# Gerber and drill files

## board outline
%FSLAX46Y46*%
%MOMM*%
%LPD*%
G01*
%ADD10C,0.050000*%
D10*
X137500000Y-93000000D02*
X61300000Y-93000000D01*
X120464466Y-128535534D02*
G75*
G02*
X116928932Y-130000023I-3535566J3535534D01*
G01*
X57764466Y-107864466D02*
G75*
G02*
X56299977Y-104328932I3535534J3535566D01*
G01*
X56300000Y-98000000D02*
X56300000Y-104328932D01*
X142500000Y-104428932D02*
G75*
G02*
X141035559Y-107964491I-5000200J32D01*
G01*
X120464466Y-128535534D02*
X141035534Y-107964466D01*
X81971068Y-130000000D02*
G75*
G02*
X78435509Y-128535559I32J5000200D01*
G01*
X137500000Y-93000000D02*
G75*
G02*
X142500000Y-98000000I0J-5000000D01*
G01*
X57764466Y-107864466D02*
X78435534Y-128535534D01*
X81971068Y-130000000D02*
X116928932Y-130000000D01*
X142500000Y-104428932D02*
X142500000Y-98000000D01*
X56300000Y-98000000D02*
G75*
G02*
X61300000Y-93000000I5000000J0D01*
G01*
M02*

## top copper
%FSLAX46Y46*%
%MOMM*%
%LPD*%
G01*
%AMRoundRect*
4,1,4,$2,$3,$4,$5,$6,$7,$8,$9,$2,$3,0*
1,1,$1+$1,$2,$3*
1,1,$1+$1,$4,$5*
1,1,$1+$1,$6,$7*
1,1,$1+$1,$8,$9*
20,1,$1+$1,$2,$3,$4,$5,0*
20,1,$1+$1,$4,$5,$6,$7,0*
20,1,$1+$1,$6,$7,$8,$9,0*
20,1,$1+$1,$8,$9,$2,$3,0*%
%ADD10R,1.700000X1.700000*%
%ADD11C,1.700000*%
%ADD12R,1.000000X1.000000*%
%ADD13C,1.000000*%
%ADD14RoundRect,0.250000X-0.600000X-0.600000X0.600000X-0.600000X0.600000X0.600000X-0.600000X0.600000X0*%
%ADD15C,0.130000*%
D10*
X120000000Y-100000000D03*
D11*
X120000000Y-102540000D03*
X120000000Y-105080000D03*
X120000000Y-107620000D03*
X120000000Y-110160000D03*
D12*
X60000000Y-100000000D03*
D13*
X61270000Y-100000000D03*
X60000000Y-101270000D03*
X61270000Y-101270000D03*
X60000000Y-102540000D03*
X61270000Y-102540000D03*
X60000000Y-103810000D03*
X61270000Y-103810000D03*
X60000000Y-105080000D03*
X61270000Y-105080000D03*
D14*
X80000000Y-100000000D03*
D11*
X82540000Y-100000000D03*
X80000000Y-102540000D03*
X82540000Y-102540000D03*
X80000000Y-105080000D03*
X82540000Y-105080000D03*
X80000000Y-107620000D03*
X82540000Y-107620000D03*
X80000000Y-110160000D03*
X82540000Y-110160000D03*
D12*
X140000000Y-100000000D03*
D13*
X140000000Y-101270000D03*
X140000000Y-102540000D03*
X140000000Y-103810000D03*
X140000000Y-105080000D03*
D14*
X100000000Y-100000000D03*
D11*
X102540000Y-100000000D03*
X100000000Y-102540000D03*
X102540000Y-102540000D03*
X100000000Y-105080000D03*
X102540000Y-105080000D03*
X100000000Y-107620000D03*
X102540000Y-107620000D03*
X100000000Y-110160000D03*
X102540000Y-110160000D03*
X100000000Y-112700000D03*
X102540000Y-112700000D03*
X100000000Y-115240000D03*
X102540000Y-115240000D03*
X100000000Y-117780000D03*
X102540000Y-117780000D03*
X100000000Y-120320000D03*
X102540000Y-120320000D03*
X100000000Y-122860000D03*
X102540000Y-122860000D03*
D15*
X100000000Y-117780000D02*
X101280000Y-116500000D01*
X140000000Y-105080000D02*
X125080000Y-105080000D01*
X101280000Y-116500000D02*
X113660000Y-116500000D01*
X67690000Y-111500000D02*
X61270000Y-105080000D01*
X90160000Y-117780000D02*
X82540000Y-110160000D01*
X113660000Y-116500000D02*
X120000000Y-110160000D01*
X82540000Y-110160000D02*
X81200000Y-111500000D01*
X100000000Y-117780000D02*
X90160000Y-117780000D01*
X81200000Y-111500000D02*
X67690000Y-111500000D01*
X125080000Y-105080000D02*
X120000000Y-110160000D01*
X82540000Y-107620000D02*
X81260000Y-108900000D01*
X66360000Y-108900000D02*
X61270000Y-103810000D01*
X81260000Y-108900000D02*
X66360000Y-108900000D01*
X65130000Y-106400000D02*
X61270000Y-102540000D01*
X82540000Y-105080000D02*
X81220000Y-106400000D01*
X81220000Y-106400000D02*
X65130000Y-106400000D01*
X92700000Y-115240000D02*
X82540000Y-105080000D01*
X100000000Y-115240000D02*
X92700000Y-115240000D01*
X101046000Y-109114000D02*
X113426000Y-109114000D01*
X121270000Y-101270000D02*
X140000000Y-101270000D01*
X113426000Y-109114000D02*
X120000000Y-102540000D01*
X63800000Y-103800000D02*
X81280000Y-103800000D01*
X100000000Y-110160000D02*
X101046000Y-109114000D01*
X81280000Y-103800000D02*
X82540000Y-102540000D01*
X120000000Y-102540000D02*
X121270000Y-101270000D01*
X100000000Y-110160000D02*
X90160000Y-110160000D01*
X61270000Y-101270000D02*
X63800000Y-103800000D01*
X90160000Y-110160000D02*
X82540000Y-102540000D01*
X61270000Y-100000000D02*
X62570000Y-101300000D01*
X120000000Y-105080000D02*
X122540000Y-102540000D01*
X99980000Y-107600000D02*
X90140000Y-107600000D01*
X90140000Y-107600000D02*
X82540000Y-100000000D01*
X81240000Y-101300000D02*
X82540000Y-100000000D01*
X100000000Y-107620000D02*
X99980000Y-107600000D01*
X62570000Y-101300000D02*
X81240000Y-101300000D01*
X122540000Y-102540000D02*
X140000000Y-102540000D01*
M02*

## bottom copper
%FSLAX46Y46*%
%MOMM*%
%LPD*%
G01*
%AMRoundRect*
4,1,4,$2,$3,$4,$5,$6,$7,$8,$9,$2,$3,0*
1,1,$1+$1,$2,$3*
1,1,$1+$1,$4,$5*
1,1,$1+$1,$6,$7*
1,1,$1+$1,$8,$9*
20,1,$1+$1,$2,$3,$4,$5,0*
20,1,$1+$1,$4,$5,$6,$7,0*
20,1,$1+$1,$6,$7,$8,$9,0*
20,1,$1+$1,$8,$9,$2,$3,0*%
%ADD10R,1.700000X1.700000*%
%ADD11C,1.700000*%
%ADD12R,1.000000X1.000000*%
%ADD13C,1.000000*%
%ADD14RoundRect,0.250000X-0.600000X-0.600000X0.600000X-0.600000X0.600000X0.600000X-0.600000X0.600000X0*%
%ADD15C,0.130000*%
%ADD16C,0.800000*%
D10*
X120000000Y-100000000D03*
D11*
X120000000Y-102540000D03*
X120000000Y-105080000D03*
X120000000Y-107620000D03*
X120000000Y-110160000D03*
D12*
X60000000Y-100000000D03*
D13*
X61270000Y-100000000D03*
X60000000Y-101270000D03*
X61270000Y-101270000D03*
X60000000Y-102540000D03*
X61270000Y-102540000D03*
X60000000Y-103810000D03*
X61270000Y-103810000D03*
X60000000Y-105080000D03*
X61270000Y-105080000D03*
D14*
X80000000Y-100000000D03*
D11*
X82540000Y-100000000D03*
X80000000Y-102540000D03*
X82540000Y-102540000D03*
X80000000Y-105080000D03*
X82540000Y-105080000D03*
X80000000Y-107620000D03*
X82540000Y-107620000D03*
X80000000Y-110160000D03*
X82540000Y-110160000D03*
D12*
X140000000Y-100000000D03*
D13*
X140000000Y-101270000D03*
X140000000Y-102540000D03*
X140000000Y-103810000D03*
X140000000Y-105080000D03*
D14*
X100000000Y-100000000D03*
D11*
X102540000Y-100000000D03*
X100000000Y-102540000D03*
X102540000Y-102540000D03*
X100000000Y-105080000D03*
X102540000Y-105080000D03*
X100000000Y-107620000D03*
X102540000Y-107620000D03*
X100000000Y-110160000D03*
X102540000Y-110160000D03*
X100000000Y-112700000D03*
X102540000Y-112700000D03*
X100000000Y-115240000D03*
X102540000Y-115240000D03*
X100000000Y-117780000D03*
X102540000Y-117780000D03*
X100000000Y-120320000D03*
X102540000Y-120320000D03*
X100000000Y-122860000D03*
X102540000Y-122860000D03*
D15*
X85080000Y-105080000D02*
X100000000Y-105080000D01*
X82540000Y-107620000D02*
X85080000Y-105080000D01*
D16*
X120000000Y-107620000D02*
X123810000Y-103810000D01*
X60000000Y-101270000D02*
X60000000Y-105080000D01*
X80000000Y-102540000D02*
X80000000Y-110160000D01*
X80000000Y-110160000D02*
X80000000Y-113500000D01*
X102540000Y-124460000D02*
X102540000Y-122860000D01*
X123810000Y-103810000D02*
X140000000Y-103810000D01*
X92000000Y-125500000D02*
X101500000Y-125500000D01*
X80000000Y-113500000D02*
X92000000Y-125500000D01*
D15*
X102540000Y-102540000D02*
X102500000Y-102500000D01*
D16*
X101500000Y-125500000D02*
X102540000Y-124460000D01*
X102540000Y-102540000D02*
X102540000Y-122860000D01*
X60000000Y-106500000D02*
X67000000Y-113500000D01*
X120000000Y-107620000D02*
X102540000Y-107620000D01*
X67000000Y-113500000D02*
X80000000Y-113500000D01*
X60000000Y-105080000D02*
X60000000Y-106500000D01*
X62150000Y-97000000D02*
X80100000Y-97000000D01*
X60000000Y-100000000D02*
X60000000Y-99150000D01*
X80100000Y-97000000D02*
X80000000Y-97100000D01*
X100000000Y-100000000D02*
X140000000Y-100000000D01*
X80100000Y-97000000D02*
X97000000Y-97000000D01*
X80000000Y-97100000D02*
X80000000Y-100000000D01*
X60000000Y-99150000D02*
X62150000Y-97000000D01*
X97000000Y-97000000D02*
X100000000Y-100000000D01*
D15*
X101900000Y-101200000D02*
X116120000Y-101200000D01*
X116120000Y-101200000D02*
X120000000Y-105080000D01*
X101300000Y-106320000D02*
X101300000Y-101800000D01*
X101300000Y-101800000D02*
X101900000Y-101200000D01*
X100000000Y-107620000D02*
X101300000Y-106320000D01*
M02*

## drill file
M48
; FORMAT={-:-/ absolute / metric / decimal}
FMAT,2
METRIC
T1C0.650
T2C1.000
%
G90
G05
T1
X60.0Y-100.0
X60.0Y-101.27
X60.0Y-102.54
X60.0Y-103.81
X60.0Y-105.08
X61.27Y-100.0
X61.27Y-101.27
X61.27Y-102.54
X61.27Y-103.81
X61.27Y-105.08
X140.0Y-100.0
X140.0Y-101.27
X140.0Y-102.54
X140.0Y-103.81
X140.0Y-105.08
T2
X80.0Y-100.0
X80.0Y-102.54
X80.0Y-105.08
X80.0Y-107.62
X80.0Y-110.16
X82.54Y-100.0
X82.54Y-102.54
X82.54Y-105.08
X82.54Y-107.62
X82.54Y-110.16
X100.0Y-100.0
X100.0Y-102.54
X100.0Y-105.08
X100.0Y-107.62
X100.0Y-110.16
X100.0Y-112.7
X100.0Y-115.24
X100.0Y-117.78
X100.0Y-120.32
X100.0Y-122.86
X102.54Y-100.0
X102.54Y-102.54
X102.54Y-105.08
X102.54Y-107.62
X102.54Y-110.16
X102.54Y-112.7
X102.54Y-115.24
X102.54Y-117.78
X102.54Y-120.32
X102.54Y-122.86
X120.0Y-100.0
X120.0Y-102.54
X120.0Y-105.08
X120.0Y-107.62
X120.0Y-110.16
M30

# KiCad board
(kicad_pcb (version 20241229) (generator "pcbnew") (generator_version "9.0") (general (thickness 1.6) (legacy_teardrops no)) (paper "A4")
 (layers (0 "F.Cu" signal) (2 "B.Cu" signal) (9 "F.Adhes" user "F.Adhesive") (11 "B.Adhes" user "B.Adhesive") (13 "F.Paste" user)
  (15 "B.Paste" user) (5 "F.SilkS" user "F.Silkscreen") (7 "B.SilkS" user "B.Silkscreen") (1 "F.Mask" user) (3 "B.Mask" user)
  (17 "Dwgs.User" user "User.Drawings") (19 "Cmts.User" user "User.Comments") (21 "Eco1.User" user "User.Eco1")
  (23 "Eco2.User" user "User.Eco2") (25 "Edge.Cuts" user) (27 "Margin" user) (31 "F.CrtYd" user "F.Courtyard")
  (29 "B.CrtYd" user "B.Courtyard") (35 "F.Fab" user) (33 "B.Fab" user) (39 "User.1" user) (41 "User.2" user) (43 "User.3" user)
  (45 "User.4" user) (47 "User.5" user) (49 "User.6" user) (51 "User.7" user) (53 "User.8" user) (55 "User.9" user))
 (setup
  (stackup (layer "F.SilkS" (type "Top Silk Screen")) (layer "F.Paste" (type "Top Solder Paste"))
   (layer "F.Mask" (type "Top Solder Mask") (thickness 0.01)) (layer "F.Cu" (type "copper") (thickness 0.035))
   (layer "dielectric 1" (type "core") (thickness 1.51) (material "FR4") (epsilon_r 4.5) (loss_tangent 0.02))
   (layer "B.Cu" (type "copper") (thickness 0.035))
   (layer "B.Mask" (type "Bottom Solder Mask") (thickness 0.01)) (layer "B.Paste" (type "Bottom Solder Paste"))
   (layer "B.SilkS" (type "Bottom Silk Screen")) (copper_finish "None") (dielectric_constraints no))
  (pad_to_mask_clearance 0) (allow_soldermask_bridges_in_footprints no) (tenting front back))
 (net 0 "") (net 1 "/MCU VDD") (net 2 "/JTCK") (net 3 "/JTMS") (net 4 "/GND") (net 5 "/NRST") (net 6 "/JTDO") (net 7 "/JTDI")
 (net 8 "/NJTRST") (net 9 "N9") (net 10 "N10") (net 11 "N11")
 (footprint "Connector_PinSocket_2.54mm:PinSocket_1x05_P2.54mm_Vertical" (layer "F.Cu") (at 120 100)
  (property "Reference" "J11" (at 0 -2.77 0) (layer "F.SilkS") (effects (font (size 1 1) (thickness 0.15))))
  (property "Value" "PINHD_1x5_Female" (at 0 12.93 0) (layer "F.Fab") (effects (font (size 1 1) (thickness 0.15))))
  (pad "1" thru_hole rect (at 0 0) (size 1.7 1.7) (drill 1) (layers "*.Cu" "*.Mask") (remove_unused_layers no) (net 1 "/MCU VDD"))
  (pad "2" thru_hole circle (at 0 2.54) (size 1.7 1.7) (drill 1) (layers "*.Cu" "*.Mask") (remove_unused_layers no) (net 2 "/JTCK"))
  (pad "3" thru_hole circle (at 0 5.08) (size 1.7 1.7) (drill 1) (layers "*.Cu" "*.Mask") (remove_unused_layers no) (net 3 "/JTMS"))
  (pad "4" thru_hole circle (at 0 7.62) (size 1.7 1.7) (drill 1) (layers "*.Cu" "*.Mask") (remove_unused_layers no) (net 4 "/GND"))
  (pad "5" thru_hole circle (at 0 10.16) (size 1.7 1.7) (drill 1) (layers "*.Cu" "*.Mask") (remove_unused_layers no) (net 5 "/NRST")))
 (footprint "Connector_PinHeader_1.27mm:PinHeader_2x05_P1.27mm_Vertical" (layer "F.Cu") (at 60 100)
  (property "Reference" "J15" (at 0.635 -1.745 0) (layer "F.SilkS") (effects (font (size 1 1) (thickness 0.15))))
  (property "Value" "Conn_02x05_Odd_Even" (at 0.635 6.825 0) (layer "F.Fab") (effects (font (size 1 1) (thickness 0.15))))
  (pad "1" thru_hole rect (at 0 0) (size 1 1) (drill 0.65) (layers "*.Cu" "*.Mask") (remove_unused_layers no) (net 1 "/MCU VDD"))
  (pad "2" thru_hole circle (at 1.27 0) (size 1 1) (drill 0.65) (layers "*.Cu" "*.Mask") (remove_unused_layers no) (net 3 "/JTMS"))
  (pad "3" thru_hole circle (at 0 1.27) (size 1 1) (drill 0.65) (layers "*.Cu" "*.Mask") (remove_unused_layers no) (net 4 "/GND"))
  (pad "4" thru_hole circle (at 1.27 1.27) (size 1 1) (drill 0.65) (layers "*.Cu" "*.Mask") (remove_unused_layers no) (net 2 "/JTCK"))
  (pad "5" thru_hole circle (at 0 2.54) (size 1 1) (drill 0.65) (layers "*.Cu" "*.Mask") (remove_unused_layers no) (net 4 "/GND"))
  (pad "6" thru_hole circle (at 1.27 2.54) (size 1 1) (drill 0.65) (layers "*.Cu" "*.Mask") (remove_unused_layers no) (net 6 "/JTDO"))
  (pad "7" thru_hole circle (at 0 3.81) (size 1 1) (drill 0.65) (layers "*.Cu" "*.Mask") (remove_unused_layers no) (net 4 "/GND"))
  (pad "8" thru_hole circle (at 1.27 3.81) (size 1 1) (drill 0.65) (layers "*.Cu" "*.Mask") (remove_unused_layers no) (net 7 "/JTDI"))
  (pad "9" thru_hole circle (at 0 5.08) (size 1 1) (drill 0.65) (layers "*.Cu" "*.Mask") (remove_unused_layers no) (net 4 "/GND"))
  (pad "10" thru_hole circle (at 1.27 5.08) (size 1 1) (drill 0.65) (layers "*.Cu" "*.Mask") (remove_unused_layers no) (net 5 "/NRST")))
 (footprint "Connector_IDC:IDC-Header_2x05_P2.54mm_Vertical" (layer "F.Cu") (at 80 100)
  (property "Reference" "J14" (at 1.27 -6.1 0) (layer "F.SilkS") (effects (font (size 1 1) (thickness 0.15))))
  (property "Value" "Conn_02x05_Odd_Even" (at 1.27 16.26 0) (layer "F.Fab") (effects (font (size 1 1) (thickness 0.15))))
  (pad "1" thru_hole roundrect (at 0 0) (size 1.7 1.7) (drill 1) (layers "*.Cu" "*.Mask") (remove_unused_layers no)
   (roundrect_rratio 0.147059) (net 1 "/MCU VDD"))
  (pad "2" thru_hole circle (at 2.54 0) (size 1.7 1.7) (drill 1) (layers "*.Cu" "*.Mask") (remove_unused_layers no) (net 3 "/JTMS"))
  (pad "3" thru_hole circle (at 0 2.54) (size 1.7 1.7) (drill 1) (layers "*.Cu" "*.Mask") (remove_unused_layers no) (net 4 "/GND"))
  (pad "4" thru_hole circle (at 2.54 2.54) (size 1.7 1.7) (drill 1) (layers "*.Cu" "*.Mask") (remove_unused_layers no) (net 2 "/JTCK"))
  (pad "5" thru_hole circle (at 0 5.08) (size 1.7 1.7) (drill 1) (layers "*.Cu" "*.Mask") (remove_unused_layers no) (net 4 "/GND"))
  (pad "6" thru_hole circle (at 2.54 5.08) (size 1.7 1.7) (drill 1) (layers "*.Cu" "*.Mask") (remove_unused_layers no) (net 6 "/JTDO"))
  (pad "7" thru_hole circle (at 0 7.62) (size 1.7 1.7) (drill 1) (layers "*.Cu" "*.Mask") (remove_unused_layers no) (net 4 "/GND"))
  (pad "8" thru_hole circle (at 2.54 7.62) (size 1.7 1.7) (drill 1) (layers "*.Cu" "*.Mask") (remove_unused_layers no) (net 7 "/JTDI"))
  (pad "9" thru_hole circle (at 0 10.16) (size 1.7 1.7) (drill 1) (layers "*.Cu" "*.Mask") (remove_unused_layers no) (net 4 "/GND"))
  (pad "10" thru_hole circle (at 2.54 10.16) (size 1.7 1.7) (drill 1) (layers "*.Cu" "*.Mask") (remove_unused_layers no) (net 5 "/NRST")))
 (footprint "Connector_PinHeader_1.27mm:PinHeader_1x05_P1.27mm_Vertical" (layer "F.Cu") (at 140 100)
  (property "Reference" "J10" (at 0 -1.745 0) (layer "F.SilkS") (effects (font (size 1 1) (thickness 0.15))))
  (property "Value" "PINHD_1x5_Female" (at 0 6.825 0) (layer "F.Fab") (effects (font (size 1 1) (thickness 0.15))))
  (pad "1" thru_hole rect (at 0 0) (size 1 1) (drill 0.65) (layers "*.Cu" "*.Mask") (remove_unused_layers no) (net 1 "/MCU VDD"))
  (pad "2" thru_hole circle (at 0 1.27) (size 1 1) (drill 0.65) (layers "*.Cu" "*.Mask") (remove_unused_layers no) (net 2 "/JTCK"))
  (pad "3" thru_hole circle (at 0 2.54) (size 1 1) (drill 0.65) (layers "*.Cu" "*.Mask") (remove_unused_layers no) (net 3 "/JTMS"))
  (pad "4" thru_hole circle (at 0 3.81) (size 1 1) (drill 0.65) (layers "*.Cu" "*.Mask") (remove_unused_layers no) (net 4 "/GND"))
  (pad "5" thru_hole circle (at 0 5.08) (size 1 1) (drill 0.65) (layers "*.Cu" "*.Mask") (remove_unused_layers no) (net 5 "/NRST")))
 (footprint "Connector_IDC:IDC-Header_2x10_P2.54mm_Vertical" (layer "F.Cu") (at 100 100)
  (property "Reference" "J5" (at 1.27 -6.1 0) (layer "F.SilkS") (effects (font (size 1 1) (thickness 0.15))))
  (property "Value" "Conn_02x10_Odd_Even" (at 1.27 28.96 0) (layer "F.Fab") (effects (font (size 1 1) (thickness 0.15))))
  (pad "1" thru_hole roundrect (at 0 0) (size 1.7 1.7) (drill 1) (layers "*.Cu" "*.Mask") (remove_unused_layers no)
   (roundrect_rratio 0.147059) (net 1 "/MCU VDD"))
  (pad "2" thru_hole circle (at 2.54 0) (size 1.7 1.7) (drill 1) (layers "*.Cu" "*.Mask") (remove_unused_layers no) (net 1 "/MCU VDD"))
  (pad "3" thru_hole circle (at 0 2.54) (size 1.7 1.7) (drill 1) (layers "*.Cu" "*.Mask") (remove_unused_layers no) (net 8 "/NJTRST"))
  (pad "4" thru_hole circle (at 2.54 2.54) (size 1.7 1.7) (drill 1) (layers "*.Cu" "*.Mask") (remove_unused_layers no) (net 4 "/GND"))
  (pad "5" thru_hole circle (at 0 5.08) (size 1.7 1.7) (drill 1) (layers "*.Cu" "*.Mask") (remove_unused_layers no) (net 7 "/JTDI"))
  (pad "6" thru_hole circle (at 2.54 5.08) (size 1.7 1.7) (drill 1) (layers "*.Cu" "*.Mask") (remove_unused_layers no) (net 4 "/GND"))
  (pad "7" thru_hole circle (at 0 7.62) (size 1.7 1.7) (drill 1) (layers "*.Cu" "*.Mask") (remove_unused_layers no) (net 3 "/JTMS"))
  (pad "8" thru_hole circle (at 2.54 7.62) (size 1.7 1.7) (drill 1) (layers "*.Cu" "*.Mask") (remove_unused_layers no) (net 4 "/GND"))
  (pad "9" thru_hole circle (at 0 10.16) (size 1.7 1.7) (drill 1) (layers "*.Cu" "*.Mask") (remove_unused_layers no) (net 2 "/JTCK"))
  (pad "10" thru_hole circle (at 2.54 10.16) (size 1.7 1.7) (drill 1) (layers "*.Cu" "*.Mask") (remove_unused_layers no) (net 4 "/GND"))
  (pad "11" thru_hole circle (at 0 12.7) (size 1.7 1.7) (drill 1) (layers "*.Cu" "*.Mask") (remove_unused_layers no) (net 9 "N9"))
  (pad "12" thru_hole circle (at 2.54 12.7) (size 1.7 1.7) (drill 1) (layers "*.Cu" "*.Mask") (remove_unused_layers no) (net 4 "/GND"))
  (pad "13" thru_hole circle (at 0 15.24) (size 1.7 1.7) (drill 1) (layers "*.Cu" "*.Mask") (remove_unused_layers no) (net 6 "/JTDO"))
  (pad "14" thru_hole circle (at 2.54 15.24) (size 1.7 1.7) (drill 1) (layers "*.Cu" "*.Mask") (remove_unused_layers no) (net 4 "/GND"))
  (pad "15" thru_hole circle (at 0 17.78) (size 1.7 1.7) (drill 1) (layers "*.Cu" "*.Mask") (remove_unused_layers no) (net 5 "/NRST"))
  (pad "16" thru_hole circle (at 2.54 17.78) (size 1.7 1.7) (drill 1) (layers "*.Cu" "*.Mask") (remove_unused_layers no) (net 4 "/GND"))
  (pad "17" thru_hole circle (at 0 20.32) (size 1.7 1.7) (drill 1) (layers "*.Cu" "*.Mask") (remove_unused_layers no) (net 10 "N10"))
  (pad "18" thru_hole circle (at 2.54 20.32) (size 1.7 1.7) (drill 1) (layers "*.Cu" "*.Mask") (remove_unused_layers no) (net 4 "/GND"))
  (pad "19" thru_hole circle (at 0 22.86) (size 1.7 1.7) (drill 1) (layers "*.Cu" "*.Mask") (remove_unused_layers no) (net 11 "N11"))
  (pad "20" thru_hole circle (at 2.54 22.86) (size 1.7 1.7) (drill 1) (layers "*.Cu" "*.Mask") (remove_unused_layers no) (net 4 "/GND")))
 (gr_line (start 137.5 93) (end 61.3 93) (stroke (width 0.05) (type default)) (layer "Edge.Cuts"))
 (gr_arc (start 120.464466 128.535534) (mid 118.842349 129.619398) (end 116.928932 130) (stroke (width 0.05) (type default))
  (layer "Edge.Cuts"))
 (gr_arc (start 57.764466 107.864466) (mid 56.680602 106.242349) (end 56.3 104.328932) (stroke (width 0.05) (type default))
  (layer "Edge.Cuts"))
 (gr_line (start 56.3 98) (end 56.3 104.328932) (stroke (width 0.05) (type default)) (layer "Edge.Cuts"))
 (gr_arc (start 142.5 104.428932) (mid 142.119387 106.342342) (end 141.035534 107.964466) (stroke (width 0.05) (type default))
  (layer "Edge.Cuts"))
 (gr_line (start 120.464466 128.535534) (end 141.035534 107.964466) (stroke (width 0.05) (type default)) (layer "Edge.Cuts"))
 (gr_arc (start 81.971068 130) (mid 80.057658 129.619387) (end 78.435534 128.535534) (stroke (width 0.05) (type default))
  (layer "Edge.Cuts"))
 (gr_arc (start 137.5 93) (mid 141.035534 94.464466) (end 142.5 98) (stroke (width 0.05) (type default)) (layer "Edge.Cuts"))
 (gr_line (start 57.764466 107.864466) (end 78.435534 128.535534) (stroke (width 0.05) (type default)) (layer "Edge.Cuts"))
 (gr_line (start 81.971068 130) (end 116.928932 130) (stroke (width 0.05) (type default)) (layer "Edge.Cuts"))
 (gr_line (start 142.5 104.428932) (end 142.5 98) (stroke (width 0.05) (type default)) (layer "Edge.Cuts"))
 (gr_arc (start 56.3 98) (mid 57.764466 94.464466) (end 61.3 93) (stroke (width 0.05) (type default)) (layer "Edge.Cuts"))
 (segment (start 100 117.78) (end 101.28 116.5) (width 0.13) (layer "F.Cu") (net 5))
 (segment (start 140 105.08) (end 125.08 105.08) (width 0.13) (layer "F.Cu") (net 5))
 (segment (start 101.28 116.5) (end 113.66 116.5) (width 0.13) (layer "F.Cu") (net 5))
 (segment (start 67.69 111.5) (end 61.27 105.08) (width 0.13) (layer "F.Cu") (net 5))
 (segment (start 90.16 117.78) (end 82.54 110.16) (width 0.13) (layer "F.Cu") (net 5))
 (segment (start 113.66 116.5) (end 120 110.16) (width 0.13) (layer "F.Cu") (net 5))
 (segment (start 82.54 110.16) (end 81.2 111.5) (width 0.13) (layer "F.Cu") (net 5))
 (segment (start 100 117.78) (end 90.16 117.78) (width 0.13) (layer "F.Cu") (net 5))
 (segment (start 81.2 111.5) (end 67.69 111.5) (width 0.13) (layer "F.Cu") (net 5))
 (segment (start 125.08 105.08) (end 120 110.16) (width 0.13) (layer "F.Cu") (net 5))
 (segment (start 82.54 107.62) (end 81.26 108.9) (width 0.13) (layer "F.Cu") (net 7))
 (segment (start 66.36 108.9) (end 61.27 103.81) (width 0.13) (layer "F.Cu") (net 7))
 (segment (start 81.26 108.9) (end 66.36 108.9) (width 0.13) (layer "F.Cu") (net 7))
 (segment (start 85.08 105.08) (end 100 105.08) (width 0.13) (layer "B.Cu") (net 7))
 (segment (start 82.54 107.62) (end 85.08 105.08) (width 0.13) (layer "B.Cu") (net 7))
 (segment (start 120 107.62) (end 123.81 103.81) (width 0.8) (layer "B.Cu") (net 4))
 (segment (start 60 101.27) (end 60 105.08) (width 0.8) (layer "B.Cu") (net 4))
 (segment (start 80 102.54) (end 80 110.16) (width 0.8) (layer "B.Cu") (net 4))
 (segment (start 80 110.16) (end 80 113.5) (width 0.8) (layer "B.Cu") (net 4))
 (segment (start 102.54 124.46) (end 102.54 122.86) (width 0.8) (layer "B.Cu") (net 4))
 (segment (start 123.81 103.81) (end 140 103.81) (width 0.8) (layer "B.Cu") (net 4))
 (segment (start 92 125.5) (end 101.5 125.5) (width 0.8) (layer "B.Cu") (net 4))
 (segment (start 80 113.5) (end 92 125.5) (width 0.8) (layer "B.Cu") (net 4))
 (segment (start 102.54 102.54) (end 102.5 102.5) (width 0.13) (layer "B.Cu") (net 4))
 (segment (start 101.5 125.5) (end 102.54 124.46) (width 0.8) (layer "B.Cu") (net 4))
 (segment (start 102.54 102.54) (end 102.54 122.86) (width 0.8) (layer "B.Cu") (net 4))
 (segment (start 60 106.5) (end 67 113.5) (width 0.8) (layer "B.Cu") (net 4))
 (segment (start 120 107.62) (end 102.54 107.62) (width 0.8) (layer "B.Cu") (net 4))
 (segment (start 67 113.5) (end 80 113.5) (width 0.8) (layer "B.Cu") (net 4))
 (segment (start 60 105.08) (end 60 106.5) (width 0.8) (layer "B.Cu") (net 4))
 (segment (start 65.13 106.4) (end 61.27 102.54) (width 0.13) (layer "F.Cu") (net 6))
 (segment (start 82.54 105.08) (end 81.22 106.4) (width 0.13) (layer "F.Cu") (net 6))
 (segment (start 81.22 106.4) (end 65.13 106.4) (width 0.13) (layer "F.Cu") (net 6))
 (segment (start 92.7 115.24) (end 82.54 105.08) (width 0.13) (layer "F.Cu") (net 6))
 (segment (start 100 115.24) (end 92.7 115.24) (width 0.13) (layer "F.Cu") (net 6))
 (segment (start 101.046 109.114) (end 113.426 109.114) (width 0.13) (layer "F.Cu") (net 2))
 (segment (start 121.27 101.27) (end 140 101.27) (width 0.13) (layer "F.Cu") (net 2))
 (segment (start 113.426 109.114) (end 120 102.54) (width 0.13) (layer "F.Cu") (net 2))
 (segment (start 63.8 103.8) (end 81.28 103.8) (width 0.13) (layer "F.Cu") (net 2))
 (segment (start 100 110.16) (end 101.046 109.114) (width 0.13) (layer "F.Cu") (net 2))
 (segment (start 81.28 103.8) (end 82.54 102.54) (width 0.13) (layer "F.Cu") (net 2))
 (segment (start 120 102.54) (end 121.27 101.27) (width 0.13) (layer "F.Cu") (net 2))
 (segment (start 100 110.16) (end 90.16 110.16) (width 0.13) (layer "F.Cu") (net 2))
 (segment (start 61.27 101.27) (end 63.8 103.8) (width 0.13) (layer "F.Cu") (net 2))
 (segment (start 90.16 110.16) (end 82.54 102.54) (width 0.13) (layer "F.Cu") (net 2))
 (segment (start 62.15 97) (end 80.1 97) (width 0.8) (layer "B.Cu") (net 1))
 (segment (start 60 100) (end 60 99.15) (width 0.8) (layer "B.Cu") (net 1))
 (segment (start 80.1 97) (end 80 97.1) (width 0.8) (layer "B.Cu") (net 1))
 (segment (start 100 100) (end 140 100) (width 0.8) (layer "B.Cu") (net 1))
 (segment (start 80.1 97) (end 97 97) (width 0.8) (layer "B.Cu") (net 1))
 (segment (start 80 97.1) (end 80 100) (width 0.8) (layer "B.Cu") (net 1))
 (segment (start 60 99.15) (end 62.15 97) (width 0.8) (layer "B.Cu") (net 1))
 (segment (start 97 97) (end 100 100) (width 0.8) (layer "B.Cu") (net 1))
 (segment (start 61.27 100) (end 62.57 101.3) (width 0.13) (layer "F.Cu") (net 3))
 (segment (start 120 105.08) (end 122.54 102.54) (width 0.13) (layer "F.Cu") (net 3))
 (segment (start 99.98 107.6) (end 90.14 107.6) (width 0.13) (layer "F.Cu") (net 3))
 (segment (start 90.14 107.6) (end 82.54 100) (width 0.13) (layer "F.Cu") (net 3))
 (segment (start 81.24 101.3) (end 82.54 100) (width 0.13) (layer "F.Cu") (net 3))
 (segment (start 100 107.62) (end 99.98 107.6) (width 0.13) (layer "F.Cu") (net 3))
 (segment (start 62.57 101.3) (end 81.24 101.3) (width 0.13) (layer "F.Cu") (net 3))
 (segment (start 122.54 102.54) (end 140 102.54) (width 0.13) (layer "F.Cu") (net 3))
 (segment (start 101.9 101.2) (end 116.12 101.2) (width 0.13) (layer "B.Cu") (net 3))
 (segment (start 116.12 101.2) (end 120 105.08) (width 0.13) (layer "B.Cu") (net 3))
 (segment (start 101.3 106.32) (end 101.3 101.8) (width 0.13) (layer "B.Cu") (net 3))
 (segment (start 101.3 101.8) (end 101.9 101.2) (width 0.13) (layer "B.Cu") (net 3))
 (segment (start 100 107.62) (end 101.3 106.32) (width 0.13) (layer "B.Cu") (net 3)))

